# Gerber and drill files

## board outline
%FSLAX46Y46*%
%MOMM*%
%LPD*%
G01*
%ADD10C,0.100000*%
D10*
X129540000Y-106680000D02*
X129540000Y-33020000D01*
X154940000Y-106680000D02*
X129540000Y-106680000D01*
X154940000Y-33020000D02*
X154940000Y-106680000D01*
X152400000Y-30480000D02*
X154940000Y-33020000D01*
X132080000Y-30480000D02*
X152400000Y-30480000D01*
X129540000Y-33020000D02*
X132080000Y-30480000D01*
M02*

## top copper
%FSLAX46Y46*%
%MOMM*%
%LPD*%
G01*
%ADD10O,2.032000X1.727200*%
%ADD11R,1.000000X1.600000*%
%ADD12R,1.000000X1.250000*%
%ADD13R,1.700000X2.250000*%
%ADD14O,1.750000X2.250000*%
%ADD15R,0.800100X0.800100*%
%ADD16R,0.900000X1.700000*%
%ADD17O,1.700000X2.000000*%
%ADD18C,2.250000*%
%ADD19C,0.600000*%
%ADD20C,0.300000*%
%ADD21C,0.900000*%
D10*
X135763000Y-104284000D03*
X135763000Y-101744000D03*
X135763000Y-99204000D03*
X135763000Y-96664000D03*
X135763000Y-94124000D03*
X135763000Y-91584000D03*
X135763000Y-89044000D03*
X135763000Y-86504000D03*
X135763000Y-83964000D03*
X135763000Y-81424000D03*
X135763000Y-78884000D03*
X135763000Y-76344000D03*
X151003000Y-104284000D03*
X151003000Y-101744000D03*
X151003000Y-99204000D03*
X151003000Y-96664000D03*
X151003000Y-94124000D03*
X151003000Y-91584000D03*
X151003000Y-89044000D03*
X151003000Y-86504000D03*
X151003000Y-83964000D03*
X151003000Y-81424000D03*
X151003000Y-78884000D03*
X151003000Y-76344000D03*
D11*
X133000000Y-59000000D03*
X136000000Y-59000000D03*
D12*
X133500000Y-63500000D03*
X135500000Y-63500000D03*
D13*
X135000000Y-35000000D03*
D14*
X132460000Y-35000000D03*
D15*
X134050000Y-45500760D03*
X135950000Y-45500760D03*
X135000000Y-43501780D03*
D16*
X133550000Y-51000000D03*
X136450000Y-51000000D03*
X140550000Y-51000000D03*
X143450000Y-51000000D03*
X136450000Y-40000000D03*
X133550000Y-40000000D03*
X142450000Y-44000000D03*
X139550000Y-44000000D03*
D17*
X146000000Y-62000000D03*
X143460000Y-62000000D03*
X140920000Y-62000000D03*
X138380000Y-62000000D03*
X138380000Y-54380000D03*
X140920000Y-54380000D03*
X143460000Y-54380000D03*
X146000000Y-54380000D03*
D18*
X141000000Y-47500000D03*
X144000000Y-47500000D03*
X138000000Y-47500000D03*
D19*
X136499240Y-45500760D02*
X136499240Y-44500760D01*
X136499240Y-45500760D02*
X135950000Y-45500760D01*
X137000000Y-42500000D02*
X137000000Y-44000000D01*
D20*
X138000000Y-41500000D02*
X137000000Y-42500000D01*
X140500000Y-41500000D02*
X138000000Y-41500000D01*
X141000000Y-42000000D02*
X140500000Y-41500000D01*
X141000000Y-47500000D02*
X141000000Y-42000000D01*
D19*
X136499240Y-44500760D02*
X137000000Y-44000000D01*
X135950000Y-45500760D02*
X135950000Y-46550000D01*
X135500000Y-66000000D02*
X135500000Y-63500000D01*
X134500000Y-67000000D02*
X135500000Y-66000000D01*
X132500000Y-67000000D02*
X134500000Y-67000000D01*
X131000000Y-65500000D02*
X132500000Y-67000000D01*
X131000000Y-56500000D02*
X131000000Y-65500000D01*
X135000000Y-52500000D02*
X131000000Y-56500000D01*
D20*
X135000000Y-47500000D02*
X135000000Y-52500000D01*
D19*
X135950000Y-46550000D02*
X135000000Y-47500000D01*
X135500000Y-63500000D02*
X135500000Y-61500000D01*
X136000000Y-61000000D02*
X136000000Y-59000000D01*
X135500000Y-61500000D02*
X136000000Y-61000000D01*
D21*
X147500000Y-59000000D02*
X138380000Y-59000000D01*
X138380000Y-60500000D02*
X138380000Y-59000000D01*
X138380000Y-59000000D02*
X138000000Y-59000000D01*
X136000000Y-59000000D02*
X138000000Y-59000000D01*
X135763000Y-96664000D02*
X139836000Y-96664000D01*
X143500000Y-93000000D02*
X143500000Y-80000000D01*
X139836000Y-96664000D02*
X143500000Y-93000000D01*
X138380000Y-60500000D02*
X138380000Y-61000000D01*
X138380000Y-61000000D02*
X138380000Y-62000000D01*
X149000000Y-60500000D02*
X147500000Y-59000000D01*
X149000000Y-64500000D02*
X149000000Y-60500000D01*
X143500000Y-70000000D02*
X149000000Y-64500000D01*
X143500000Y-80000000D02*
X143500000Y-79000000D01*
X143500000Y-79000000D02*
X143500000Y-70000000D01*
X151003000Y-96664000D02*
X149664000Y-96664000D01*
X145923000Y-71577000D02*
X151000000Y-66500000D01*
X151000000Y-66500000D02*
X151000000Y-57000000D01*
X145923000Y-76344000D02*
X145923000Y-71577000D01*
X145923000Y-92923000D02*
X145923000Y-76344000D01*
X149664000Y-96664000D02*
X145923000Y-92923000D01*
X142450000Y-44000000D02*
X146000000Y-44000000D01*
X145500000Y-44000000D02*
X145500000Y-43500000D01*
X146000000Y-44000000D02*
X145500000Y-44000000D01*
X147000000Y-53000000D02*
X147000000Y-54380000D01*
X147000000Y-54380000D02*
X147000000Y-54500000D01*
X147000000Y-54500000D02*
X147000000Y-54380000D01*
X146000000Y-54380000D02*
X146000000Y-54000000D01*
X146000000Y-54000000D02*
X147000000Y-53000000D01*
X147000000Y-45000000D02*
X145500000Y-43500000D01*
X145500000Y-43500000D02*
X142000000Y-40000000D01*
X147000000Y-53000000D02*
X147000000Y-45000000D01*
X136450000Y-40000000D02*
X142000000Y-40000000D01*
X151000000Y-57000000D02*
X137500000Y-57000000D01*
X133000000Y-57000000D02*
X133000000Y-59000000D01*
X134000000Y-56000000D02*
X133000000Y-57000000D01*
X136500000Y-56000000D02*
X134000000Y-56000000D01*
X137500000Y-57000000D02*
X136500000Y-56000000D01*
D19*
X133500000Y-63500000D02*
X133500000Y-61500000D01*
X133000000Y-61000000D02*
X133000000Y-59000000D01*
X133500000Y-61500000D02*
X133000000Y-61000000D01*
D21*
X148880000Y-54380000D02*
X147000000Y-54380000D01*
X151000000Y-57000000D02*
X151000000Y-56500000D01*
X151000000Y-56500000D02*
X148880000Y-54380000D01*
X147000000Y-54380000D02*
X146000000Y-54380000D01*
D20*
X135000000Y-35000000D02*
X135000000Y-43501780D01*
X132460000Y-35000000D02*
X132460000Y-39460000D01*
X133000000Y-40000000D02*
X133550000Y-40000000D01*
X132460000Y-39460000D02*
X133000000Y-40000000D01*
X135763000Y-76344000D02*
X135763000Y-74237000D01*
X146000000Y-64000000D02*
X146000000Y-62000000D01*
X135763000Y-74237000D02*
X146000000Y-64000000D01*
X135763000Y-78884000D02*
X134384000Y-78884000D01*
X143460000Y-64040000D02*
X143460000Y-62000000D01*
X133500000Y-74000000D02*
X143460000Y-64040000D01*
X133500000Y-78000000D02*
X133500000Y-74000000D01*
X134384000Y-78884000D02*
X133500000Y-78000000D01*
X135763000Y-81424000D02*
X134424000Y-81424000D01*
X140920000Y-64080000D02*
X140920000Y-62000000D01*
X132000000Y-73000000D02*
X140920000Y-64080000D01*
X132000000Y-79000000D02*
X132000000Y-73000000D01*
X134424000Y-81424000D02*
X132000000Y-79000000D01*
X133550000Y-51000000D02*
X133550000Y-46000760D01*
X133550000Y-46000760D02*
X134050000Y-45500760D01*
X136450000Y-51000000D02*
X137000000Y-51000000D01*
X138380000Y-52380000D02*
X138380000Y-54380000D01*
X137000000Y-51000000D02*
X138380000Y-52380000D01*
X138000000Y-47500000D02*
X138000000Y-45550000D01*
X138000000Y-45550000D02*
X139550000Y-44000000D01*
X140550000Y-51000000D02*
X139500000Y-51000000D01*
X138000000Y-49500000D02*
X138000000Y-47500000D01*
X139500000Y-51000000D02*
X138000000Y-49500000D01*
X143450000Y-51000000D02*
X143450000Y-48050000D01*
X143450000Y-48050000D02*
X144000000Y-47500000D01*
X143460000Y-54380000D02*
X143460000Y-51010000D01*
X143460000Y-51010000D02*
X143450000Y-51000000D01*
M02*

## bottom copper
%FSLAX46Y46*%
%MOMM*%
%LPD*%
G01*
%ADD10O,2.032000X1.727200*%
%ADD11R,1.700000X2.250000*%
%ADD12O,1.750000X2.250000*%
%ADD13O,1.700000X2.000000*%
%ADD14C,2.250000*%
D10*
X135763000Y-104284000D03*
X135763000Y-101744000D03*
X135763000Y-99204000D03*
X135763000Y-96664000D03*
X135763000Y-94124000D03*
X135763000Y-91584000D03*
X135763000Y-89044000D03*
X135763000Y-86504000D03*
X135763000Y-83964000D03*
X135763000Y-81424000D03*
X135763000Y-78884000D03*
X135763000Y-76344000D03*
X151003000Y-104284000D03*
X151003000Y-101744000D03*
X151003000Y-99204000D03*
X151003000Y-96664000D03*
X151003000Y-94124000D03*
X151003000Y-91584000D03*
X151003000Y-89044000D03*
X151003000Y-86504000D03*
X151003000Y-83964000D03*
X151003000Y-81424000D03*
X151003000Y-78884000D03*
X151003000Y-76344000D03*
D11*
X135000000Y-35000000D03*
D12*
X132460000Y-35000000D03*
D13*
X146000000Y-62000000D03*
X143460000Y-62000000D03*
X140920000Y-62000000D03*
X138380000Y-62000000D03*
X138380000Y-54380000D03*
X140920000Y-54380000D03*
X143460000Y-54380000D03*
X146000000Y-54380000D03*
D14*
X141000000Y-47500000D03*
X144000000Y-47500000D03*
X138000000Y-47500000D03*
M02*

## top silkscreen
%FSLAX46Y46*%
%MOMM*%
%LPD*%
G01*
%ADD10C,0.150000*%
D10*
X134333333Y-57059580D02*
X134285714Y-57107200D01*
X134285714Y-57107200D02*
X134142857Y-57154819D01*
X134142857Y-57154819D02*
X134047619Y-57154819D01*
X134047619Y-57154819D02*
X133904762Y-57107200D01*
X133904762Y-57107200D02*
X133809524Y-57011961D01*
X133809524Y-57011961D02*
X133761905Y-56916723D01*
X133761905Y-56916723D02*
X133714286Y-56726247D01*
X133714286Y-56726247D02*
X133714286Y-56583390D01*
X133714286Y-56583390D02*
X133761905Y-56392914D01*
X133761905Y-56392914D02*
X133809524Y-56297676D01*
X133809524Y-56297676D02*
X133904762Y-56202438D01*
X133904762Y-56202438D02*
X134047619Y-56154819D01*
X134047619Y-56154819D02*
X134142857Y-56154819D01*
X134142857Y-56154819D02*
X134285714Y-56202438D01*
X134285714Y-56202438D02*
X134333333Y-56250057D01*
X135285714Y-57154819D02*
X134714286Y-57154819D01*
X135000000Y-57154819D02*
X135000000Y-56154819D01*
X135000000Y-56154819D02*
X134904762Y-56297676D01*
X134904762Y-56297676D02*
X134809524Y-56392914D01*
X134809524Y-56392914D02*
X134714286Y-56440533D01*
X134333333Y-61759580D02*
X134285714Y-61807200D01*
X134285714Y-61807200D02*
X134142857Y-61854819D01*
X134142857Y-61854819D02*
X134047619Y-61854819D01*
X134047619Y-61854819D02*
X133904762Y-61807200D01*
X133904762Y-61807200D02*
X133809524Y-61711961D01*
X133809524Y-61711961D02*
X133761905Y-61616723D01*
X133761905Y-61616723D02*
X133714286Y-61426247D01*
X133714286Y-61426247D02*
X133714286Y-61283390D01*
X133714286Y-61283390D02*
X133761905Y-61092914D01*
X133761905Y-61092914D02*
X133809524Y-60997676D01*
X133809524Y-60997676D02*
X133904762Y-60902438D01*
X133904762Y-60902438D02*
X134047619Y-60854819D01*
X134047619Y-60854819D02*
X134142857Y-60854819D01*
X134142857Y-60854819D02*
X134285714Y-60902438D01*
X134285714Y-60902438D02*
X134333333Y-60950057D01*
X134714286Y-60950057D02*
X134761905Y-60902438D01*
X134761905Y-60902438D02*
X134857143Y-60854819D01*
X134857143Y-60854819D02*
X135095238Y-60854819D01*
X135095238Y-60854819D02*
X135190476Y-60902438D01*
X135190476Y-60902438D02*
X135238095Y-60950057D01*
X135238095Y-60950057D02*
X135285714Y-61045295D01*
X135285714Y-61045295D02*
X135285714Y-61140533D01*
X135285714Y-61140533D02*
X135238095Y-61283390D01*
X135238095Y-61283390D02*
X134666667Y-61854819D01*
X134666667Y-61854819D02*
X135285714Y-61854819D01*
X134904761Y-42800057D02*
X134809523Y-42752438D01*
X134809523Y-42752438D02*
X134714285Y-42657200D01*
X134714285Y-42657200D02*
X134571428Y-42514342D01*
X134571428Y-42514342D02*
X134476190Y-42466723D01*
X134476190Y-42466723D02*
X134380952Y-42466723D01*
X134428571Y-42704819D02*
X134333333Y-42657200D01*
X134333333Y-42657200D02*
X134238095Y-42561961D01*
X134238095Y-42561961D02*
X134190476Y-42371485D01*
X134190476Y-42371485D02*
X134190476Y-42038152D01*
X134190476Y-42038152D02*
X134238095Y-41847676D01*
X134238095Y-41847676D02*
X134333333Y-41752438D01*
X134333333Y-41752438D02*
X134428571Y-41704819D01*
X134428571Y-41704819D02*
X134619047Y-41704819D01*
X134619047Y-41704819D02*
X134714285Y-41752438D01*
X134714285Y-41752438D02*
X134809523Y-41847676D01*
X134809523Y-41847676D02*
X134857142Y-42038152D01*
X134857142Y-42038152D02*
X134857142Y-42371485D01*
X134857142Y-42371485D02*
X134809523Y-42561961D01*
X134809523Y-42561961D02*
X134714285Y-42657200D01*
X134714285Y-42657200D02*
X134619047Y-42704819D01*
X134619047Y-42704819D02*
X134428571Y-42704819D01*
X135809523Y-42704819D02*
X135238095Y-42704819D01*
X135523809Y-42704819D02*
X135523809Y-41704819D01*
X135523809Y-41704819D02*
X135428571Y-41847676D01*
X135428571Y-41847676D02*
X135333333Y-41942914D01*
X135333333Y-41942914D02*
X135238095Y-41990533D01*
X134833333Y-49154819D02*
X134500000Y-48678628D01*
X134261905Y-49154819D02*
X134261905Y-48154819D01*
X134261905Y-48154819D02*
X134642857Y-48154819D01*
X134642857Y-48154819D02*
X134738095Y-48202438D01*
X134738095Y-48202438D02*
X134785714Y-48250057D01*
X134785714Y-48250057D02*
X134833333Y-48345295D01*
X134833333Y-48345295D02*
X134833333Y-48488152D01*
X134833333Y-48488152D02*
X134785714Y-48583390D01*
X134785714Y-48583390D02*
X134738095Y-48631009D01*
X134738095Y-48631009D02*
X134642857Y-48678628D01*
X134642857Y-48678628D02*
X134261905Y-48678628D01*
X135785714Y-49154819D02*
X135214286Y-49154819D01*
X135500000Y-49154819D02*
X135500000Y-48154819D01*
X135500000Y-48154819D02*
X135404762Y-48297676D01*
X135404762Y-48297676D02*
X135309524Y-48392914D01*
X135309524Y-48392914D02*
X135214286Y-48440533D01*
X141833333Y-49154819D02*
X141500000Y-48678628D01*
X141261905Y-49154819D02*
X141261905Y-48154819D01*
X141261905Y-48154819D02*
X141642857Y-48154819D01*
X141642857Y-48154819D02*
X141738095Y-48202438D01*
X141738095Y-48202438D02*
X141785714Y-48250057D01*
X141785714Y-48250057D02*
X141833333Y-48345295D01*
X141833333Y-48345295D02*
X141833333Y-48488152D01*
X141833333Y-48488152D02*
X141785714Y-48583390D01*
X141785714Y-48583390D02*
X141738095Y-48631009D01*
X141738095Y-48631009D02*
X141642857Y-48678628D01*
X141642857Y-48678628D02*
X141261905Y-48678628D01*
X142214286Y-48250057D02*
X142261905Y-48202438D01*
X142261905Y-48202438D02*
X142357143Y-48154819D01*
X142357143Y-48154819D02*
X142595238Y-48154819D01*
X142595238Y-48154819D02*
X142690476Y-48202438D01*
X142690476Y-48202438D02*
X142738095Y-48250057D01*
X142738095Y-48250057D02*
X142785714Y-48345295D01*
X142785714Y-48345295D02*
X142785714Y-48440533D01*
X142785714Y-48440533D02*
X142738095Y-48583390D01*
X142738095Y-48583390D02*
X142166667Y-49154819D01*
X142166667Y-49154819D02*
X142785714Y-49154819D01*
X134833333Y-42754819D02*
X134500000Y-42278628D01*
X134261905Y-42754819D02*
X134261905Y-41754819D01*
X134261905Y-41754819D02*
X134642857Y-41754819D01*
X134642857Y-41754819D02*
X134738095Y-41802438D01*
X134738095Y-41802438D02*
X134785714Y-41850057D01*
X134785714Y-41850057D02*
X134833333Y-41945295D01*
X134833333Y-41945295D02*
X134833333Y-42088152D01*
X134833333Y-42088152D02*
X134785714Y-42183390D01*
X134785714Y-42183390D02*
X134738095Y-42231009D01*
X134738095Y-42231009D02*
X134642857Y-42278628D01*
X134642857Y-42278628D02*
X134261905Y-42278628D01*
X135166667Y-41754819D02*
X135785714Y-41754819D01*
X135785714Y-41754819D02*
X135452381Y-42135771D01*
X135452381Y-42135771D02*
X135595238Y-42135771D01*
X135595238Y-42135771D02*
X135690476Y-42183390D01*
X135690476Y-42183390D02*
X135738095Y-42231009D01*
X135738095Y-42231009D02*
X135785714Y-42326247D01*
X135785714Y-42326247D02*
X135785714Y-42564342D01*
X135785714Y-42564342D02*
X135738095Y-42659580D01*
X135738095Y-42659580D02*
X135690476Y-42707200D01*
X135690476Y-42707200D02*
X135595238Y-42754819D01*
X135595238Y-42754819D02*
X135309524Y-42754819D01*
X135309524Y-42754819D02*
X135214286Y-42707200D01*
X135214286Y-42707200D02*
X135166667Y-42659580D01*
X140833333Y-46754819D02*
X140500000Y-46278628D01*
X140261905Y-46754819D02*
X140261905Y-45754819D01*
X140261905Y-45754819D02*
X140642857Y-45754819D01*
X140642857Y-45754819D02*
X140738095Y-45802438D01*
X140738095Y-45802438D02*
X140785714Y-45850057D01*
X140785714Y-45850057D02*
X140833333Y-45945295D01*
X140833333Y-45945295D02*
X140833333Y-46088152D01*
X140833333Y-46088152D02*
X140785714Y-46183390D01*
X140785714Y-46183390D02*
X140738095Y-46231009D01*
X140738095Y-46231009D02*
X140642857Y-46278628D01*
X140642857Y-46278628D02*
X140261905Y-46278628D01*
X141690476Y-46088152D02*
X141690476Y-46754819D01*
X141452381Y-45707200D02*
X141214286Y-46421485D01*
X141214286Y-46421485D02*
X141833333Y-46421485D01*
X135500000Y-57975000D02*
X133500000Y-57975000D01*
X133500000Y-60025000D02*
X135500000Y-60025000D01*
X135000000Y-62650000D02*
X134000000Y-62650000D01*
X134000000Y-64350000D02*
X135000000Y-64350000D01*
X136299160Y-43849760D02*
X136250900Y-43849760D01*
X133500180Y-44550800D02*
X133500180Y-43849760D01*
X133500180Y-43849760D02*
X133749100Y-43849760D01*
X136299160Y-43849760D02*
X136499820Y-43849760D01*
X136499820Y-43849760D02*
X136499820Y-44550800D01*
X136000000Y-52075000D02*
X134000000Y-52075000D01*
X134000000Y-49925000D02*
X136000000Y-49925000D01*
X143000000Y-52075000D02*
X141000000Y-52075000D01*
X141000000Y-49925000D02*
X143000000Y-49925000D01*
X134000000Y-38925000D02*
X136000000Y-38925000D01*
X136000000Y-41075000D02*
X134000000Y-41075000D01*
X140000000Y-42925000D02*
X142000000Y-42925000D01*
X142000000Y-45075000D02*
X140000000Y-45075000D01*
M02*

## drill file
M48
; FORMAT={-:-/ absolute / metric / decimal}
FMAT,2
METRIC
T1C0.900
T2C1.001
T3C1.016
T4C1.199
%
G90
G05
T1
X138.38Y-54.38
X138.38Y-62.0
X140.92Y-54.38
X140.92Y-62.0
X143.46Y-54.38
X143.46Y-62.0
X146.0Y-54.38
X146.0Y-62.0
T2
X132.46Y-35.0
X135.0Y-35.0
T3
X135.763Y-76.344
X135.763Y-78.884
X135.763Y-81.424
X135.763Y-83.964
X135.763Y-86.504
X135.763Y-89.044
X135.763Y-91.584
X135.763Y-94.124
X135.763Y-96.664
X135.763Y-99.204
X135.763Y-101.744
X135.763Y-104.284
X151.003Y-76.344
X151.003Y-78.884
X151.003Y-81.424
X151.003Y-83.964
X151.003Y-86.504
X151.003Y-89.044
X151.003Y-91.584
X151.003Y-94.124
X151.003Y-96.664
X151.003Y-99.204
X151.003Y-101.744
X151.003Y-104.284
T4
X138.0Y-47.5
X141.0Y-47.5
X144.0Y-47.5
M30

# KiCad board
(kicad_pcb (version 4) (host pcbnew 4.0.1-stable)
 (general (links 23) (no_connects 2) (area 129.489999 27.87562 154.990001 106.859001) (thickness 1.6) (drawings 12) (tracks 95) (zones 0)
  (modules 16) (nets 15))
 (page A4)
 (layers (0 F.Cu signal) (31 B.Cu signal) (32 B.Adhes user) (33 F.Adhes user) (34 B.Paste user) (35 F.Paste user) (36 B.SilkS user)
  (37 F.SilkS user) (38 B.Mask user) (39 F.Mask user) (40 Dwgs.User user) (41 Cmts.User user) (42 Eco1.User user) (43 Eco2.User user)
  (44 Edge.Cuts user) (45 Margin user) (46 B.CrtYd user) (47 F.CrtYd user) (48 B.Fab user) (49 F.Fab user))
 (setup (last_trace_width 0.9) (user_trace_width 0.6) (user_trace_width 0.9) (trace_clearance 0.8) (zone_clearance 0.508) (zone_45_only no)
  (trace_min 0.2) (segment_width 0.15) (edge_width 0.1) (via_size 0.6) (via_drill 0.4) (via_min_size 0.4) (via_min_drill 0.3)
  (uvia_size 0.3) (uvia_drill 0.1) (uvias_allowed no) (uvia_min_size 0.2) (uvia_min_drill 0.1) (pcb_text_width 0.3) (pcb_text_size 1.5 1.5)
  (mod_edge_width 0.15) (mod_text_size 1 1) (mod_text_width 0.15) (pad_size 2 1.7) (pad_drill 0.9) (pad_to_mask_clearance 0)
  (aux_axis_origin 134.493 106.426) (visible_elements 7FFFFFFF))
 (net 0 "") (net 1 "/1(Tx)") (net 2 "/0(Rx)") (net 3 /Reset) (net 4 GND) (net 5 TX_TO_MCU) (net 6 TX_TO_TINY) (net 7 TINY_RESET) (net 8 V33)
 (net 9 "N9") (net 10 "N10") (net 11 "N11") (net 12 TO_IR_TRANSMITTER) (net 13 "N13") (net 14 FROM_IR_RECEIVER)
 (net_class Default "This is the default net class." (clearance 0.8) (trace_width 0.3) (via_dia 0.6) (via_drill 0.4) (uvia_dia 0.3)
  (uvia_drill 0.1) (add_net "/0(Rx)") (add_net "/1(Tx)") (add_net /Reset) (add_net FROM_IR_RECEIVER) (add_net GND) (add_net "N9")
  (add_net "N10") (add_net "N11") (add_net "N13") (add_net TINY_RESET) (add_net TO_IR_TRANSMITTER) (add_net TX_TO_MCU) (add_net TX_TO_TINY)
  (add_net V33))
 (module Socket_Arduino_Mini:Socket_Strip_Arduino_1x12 (layer B.Cu) (at 135.763 104.284 90)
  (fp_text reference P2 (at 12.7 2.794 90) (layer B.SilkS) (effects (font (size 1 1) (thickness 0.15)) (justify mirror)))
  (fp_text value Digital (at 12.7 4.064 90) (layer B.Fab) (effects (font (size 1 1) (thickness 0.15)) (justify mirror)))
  (pad 1 thru_hole oval (at 0 0 90) (size 1.7272 2.032) (drill 1.016) (layers *.Cu *.Mask B.SilkS) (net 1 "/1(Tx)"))
  (pad 2 thru_hole oval (at 2.54 0 90) (size 1.7272 2.032) (drill 1.016) (layers *.Cu *.Mask B.SilkS) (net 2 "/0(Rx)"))
  (pad 3 thru_hole oval (at 5.08 0 90) (size 1.7272 2.032) (drill 1.016) (layers *.Cu *.Mask B.SilkS) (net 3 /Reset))
  (pad 4 thru_hole oval (at 7.62 0 90) (size 1.7272 2.032) (drill 1.016) (layers *.Cu *.Mask B.SilkS) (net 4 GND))
  (pad 5 thru_hole oval (at 10.16 0 90) (size 1.7272 2.032) (drill 1.016) (layers *.Cu *.Mask B.SilkS))
  (pad 6 thru_hole oval (at 12.7 0 90) (size 1.7272 2.032) (drill 1.016) (layers *.Cu *.Mask B.SilkS))
  (pad 7 thru_hole oval (at 15.24 0 90) (size 1.7272 2.032) (drill 1.016) (layers *.Cu *.Mask B.SilkS))
  (pad 8 thru_hole oval (at 17.78 0 90) (size 1.7272 2.032) (drill 1.016) (layers *.Cu *.Mask B.SilkS))
  (pad 9 thru_hole oval (at 20.32 0 90) (size 1.7272 2.032) (drill 1.016) (layers *.Cu *.Mask B.SilkS))
  (pad 10 thru_hole oval (at 22.86 0 90) (size 1.7272 2.032) (drill 1.016) (layers *.Cu *.Mask B.SilkS) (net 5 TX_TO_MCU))
  (pad 11 thru_hole oval (at 25.4 0 90) (size 1.7272 2.032) (drill 1.016) (layers *.Cu *.Mask B.SilkS) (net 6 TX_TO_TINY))
  (pad 12 thru_hole oval (at 27.94 0 90) (size 1.7272 2.032) (drill 1.016) (layers *.Cu *.Mask B.SilkS) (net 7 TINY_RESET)))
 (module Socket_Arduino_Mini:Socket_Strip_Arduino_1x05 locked (layer B.Cu) (at 138.303 104.284)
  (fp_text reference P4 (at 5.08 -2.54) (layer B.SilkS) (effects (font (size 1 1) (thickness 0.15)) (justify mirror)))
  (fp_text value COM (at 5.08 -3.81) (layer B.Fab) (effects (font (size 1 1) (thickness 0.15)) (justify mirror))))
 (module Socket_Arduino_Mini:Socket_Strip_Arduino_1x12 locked (layer B.Cu) (at 151.003 104.284 90)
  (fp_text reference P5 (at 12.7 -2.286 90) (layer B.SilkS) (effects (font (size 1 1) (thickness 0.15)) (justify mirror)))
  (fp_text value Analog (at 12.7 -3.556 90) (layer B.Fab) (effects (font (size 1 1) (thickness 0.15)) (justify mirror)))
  (pad 1 thru_hole oval (at 0 0 90) (size 1.7272 2.032) (drill 1.016) (layers *.Cu *.Mask B.SilkS))
  (pad 2 thru_hole oval (at 2.54 0 90) (size 1.7272 2.032) (drill 1.016) (layers *.Cu *.Mask B.SilkS) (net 4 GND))
  (pad 3 thru_hole oval (at 5.08 0 90) (size 1.7272 2.032) (drill 1.016) (layers *.Cu *.Mask B.SilkS) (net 3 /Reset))
  (pad 4 thru_hole oval (at 7.62 0 90) (size 1.7272 2.032) (drill 1.016) (layers *.Cu *.Mask B.SilkS) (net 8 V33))
  (pad 5 thru_hole oval (at 10.16 0 90) (size 1.7272 2.032) (drill 1.016) (layers *.Cu *.Mask B.SilkS))
  (pad 6 thru_hole oval (at 12.7 0 90) (size 1.7272 2.032) (drill 1.016) (layers *.Cu *.Mask B.SilkS))
  (pad 7 thru_hole oval (at 15.24 0 90) (size 1.7272 2.032) (drill 1.016) (layers *.Cu *.Mask B.SilkS))
  (pad 8 thru_hole oval (at 17.78 0 90) (size 1.7272 2.032) (drill 1.016) (layers *.Cu *.Mask B.SilkS))
  (pad 9 thru_hole oval (at 20.32 0 90) (size 1.7272 2.032) (drill 1.016) (layers *.Cu *.Mask B.SilkS))
  (pad 10 thru_hole oval (at 22.86 0 90) (size 1.7272 2.032) (drill 1.016) (layers *.Cu *.Mask B.SilkS))
  (pad 11 thru_hole oval (at 25.4 0 90) (size 1.7272 2.032) (drill 1.016) (layers *.Cu *.Mask B.SilkS))
  (pad 12 thru_hole oval (at 27.94 0 90) (size 1.7272 2.032) (drill 1.016) (layers *.Cu *.Mask B.SilkS)))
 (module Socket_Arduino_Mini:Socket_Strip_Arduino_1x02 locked (layer B.Cu) (at 138.303 78.884 90)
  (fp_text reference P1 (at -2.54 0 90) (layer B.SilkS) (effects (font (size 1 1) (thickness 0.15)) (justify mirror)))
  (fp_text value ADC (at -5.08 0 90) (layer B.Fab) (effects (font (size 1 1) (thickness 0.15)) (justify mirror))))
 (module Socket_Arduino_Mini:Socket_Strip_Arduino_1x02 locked (layer B.Cu) (at 140.843 78.884 90)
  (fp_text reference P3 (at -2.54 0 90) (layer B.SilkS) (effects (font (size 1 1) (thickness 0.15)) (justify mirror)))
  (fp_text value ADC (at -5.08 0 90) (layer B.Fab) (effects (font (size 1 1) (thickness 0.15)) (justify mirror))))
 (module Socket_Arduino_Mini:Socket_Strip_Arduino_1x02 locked (layer B.Cu) (at 145.923 76.344)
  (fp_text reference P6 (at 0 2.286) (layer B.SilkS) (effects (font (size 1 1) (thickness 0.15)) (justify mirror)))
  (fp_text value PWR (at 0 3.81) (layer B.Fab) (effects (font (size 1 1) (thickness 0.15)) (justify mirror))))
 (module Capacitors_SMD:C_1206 (layer F.Cu) (at 134.5 59)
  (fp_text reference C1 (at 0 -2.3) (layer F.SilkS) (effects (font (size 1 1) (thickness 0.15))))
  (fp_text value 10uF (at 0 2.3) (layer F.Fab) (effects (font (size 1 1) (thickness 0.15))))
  (fp_line (start 1 -1.025) (end -1 -1.025) (layer F.SilkS) (width 0.15))
  (fp_line (start -1 1.025) (end 1 1.025) (layer F.SilkS) (width 0.15))
  (pad 1 smd rect (at -1.5 0) (size 1 1.6) (layers F.Cu F.Paste F.Mask) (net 8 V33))
  (pad 2 smd rect (at 1.5 0) (size 1 1.6) (layers F.Cu F.Paste F.Mask) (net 4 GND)))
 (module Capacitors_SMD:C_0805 (layer F.Cu) (at 134.5 63.5)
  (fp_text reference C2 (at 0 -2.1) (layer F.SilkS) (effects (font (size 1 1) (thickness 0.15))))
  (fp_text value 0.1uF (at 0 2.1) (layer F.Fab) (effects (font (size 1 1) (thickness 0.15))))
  (fp_line (start 0.5 -0.85) (end -0.5 -0.85) (layer F.SilkS) (width 0.15))
  (fp_line (start -0.5 0.85) (end 0.5 0.85) (layer F.SilkS) (width 0.15))
  (pad 1 smd rect (at -1 0) (size 1 1.25) (layers F.Cu F.Paste F.Mask) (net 8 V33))
  (pad 2 smd rect (at 1 0) (size 1 1.25) (layers F.Cu F.Paste F.Mask) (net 4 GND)))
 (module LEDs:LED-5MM (layer B.Cu) (at 135 35 180)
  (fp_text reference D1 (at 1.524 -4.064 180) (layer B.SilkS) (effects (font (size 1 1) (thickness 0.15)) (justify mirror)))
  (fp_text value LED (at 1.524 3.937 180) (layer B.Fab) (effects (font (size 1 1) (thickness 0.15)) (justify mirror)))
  (pad 1 thru_hole rect (at 0 0 90) (size 2.25 1.7) (drill 1.00076) (layers *.Cu *.Mask B.SilkS) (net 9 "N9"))
  (pad 2 thru_hole oval (at 2.54 0 180) (size 1.75 2.25) (drill 1.00076) (layers *.Cu *.Mask B.SilkS) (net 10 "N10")))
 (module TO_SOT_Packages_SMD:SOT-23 (layer F.Cu) (at 135 44.5)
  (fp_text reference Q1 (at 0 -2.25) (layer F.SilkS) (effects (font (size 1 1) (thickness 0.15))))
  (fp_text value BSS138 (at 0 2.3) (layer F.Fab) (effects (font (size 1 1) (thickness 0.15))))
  (fp_line (start 1.29916 -0.65024) (end 1.2509 -0.65024) (layer F.SilkS) (width 0.15))
  (fp_line (start -1.49982 0.0508) (end -1.49982 -0.65024) (layer F.SilkS) (width 0.15))
  (fp_line (start -1.49982 -0.65024) (end -1.2509 -0.65024) (layer F.SilkS) (width 0.15))
  (fp_line (start 1.29916 -0.65024) (end 1.49982 -0.65024) (layer F.SilkS) (width 0.15))
  (fp_line (start 1.49982 -0.65024) (end 1.49982 0.0508) (layer F.SilkS) (width 0.15))
  (pad 1 smd rect (at -0.95 1.00076) (size 0.8001 0.8001) (layers F.Cu F.Paste F.Mask) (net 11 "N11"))
  (pad 2 smd rect (at 0.95 1.00076) (size 0.8001 0.8001) (layers F.Cu F.Paste F.Mask) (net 4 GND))
  (pad 3 smd rect (at 0 -0.99822) (size 0.8001 0.8001) (layers F.Cu F.Paste F.Mask) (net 9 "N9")))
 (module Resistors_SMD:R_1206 (layer F.Cu) (at 135 51)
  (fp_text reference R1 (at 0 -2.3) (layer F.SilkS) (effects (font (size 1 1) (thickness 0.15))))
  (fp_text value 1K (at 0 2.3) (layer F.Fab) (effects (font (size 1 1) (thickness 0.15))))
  (fp_line (start 1 1.075) (end -1 1.075) (layer F.SilkS) (width 0.15))
  (fp_line (start -1 -1.075) (end 1 -1.075) (layer F.SilkS) (width 0.15))
  (pad 1 smd rect (at -1.45 0) (size 0.9 1.7) (layers F.Cu F.Paste F.Mask) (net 11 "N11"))
  (pad 2 smd rect (at 1.45 0) (size 0.9 1.7) (layers F.Cu F.Paste F.Mask) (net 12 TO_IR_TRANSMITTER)))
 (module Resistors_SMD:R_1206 (layer F.Cu) (at 142 51)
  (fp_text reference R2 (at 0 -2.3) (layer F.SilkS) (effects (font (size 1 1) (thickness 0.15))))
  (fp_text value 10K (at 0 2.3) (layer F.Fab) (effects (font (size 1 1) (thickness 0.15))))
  (fp_line (start 1 1.075) (end -1 1.075) (layer F.SilkS) (width 0.15))
  (fp_line (start -1 -1.075) (end 1 -1.075) (layer F.SilkS) (width 0.15))
  (pad 1 smd rect (at -1.45 0) (size 0.9 1.7) (layers F.Cu F.Paste F.Mask) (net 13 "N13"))
  (pad 2 smd rect (at 1.45 0) (size 0.9 1.7) (layers F.Cu F.Paste F.Mask) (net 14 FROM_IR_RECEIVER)))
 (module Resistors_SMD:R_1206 (layer F.Cu) (at 135 40 180)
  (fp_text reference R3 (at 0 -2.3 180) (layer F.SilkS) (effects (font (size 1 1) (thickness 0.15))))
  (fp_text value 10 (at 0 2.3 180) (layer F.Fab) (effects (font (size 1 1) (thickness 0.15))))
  (fp_line (start 1 1.075) (end -1 1.075) (layer F.SilkS) (width 0.15))
  (fp_line (start -1 -1.075) (end 1 -1.075) (layer F.SilkS) (width 0.15))
  (pad 1 smd rect (at -1.45 0 180) (size 0.9 1.7) (layers F.Cu F.Paste F.Mask) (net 8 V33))
  (pad 2 smd rect (at 1.45 0 180) (size 0.9 1.7) (layers F.Cu F.Paste F.Mask) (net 10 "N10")))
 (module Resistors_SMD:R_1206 (layer F.Cu) (at 141 44 180)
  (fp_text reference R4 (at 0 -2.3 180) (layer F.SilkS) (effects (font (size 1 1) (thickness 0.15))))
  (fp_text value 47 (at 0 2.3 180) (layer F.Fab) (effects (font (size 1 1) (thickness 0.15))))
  (fp_line (start 1 1.075) (end -1 1.075) (layer F.SilkS) (width 0.15))
  (fp_line (start -1 -1.075) (end 1 -1.075) (layer F.SilkS) (width 0.15))
  (pad 1 smd rect (at -1.45 0 180) (size 0.9 1.7) (layers F.Cu F.Paste F.Mask) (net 8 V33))
  (pad 2 smd rect (at 1.45 0 180) (size 0.9 1.7) (layers F.Cu F.Paste F.Mask) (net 13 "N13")))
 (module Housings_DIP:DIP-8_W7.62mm (layer B.Cu) (at 146 62 90)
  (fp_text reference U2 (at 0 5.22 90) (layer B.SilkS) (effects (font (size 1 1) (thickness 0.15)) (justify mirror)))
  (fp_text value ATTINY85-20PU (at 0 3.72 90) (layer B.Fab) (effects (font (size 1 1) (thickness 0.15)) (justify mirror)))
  (pad 1 thru_hole oval (at 0 0 90) (size 2 1.7) (drill 0.9) (layers *.Cu *.Mask B.SilkS) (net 7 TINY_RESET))
  (pad 2 thru_hole oval (at 0 -2.54 90) (size 2 1.7) (drill 0.9) (layers *.Cu *.Mask B.SilkS) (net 6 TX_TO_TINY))
  (pad 3 thru_hole oval (at 0 -5.08 90) (size 2 1.7) (drill 0.9) (layers *.Cu *.Mask B.SilkS) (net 5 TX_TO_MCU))
  (pad 4 thru_hole oval (at 0 -7.62 90) (size 2 1.7) (drill 0.9) (layers *.Cu *.Mask B.SilkS) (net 4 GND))
  (pad 5 thru_hole oval (at 7.62 -7.62 90) (size 2 1.7) (drill 0.9) (layers *.Cu *.Mask B.SilkS) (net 12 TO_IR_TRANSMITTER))
  (pad 6 thru_hole oval (at 7.62 -5.08 90) (size 2 1.7) (drill 0.9) (layers *.Cu *.Mask B.SilkS))
  (pad 7 thru_hole oval (at 7.62 -2.54 90) (size 2 1.7) (drill 0.9) (layers *.Cu *.Mask B.SilkS) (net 14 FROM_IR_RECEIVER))
  (pad 8 thru_hole oval (at 7.62 0 90) (size 2 1.7) (drill 0.9) (layers *.Cu *.Mask B.SilkS) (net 8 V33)))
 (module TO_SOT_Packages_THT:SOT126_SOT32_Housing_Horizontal (layer B.Cu) (at 141 47.5 180)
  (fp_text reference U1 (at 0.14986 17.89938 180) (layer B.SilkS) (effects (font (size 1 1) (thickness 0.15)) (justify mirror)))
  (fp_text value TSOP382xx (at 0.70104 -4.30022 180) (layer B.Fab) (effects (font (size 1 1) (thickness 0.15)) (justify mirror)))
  (pad 2 thru_hole circle (at 0 0 180) (size 2.25 2.25) (drill 1.19888) (layers *.Cu *.Mask B.SilkS) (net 4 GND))
  (pad 1 thru_hole circle (at -3 0 180) (size 2.25 2.25) (drill 1.19888) (layers *.Cu *.Mask B.SilkS) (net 14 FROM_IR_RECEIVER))
  (pad 3 thru_hole circle (at 3 0 180) (size 2.25 2.25) (drill 1.19888) (layers *.Cu *.Mask B.SilkS) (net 13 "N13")))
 (gr_line (start 129.54 106.68) (end 129.54 33.02) (angle 90) (layer Edge.Cuts) (width 0.1))
 (gr_line (start 154.94 106.68) (end 129.54 106.68) (angle 90) (layer Edge.Cuts) (width 0.1))
 (gr_line (start 154.94 33.02) (end 154.94 106.68) (angle 90) (layer Edge.Cuts) (width 0.1))
 (gr_line (start 152.4 30.48) (end 154.94 33.02) (angle 90) (layer Edge.Cuts) (width 0.1))
 (gr_line (start 132.08 30.48) (end 152.4 30.48) (angle 90) (layer Edge.Cuts) (width 0.1))
 (gr_line (start 129.54 33.02) (end 132.08 30.48) (angle 90) (layer Edge.Cuts) (width 0.1))
 (segment (start 136.49924 45.50076) (end 136.49924 44.50076) (width 0.6) (layer F.Cu) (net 4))
 (segment (start 136.49924 45.50076) (end 135.95 45.50076) (width 0.6) (layer F.Cu) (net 4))
 (segment (start 137 42.5) (end 137 44) (width 0.6) (layer F.Cu) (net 4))
 (segment (start 138 41.5) (end 137 42.5) (width 0.3) (layer F.Cu) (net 4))
 (segment (start 140.5 41.5) (end 138 41.5) (width 0.3) (layer F.Cu) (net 4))
 (segment (start 141 42) (end 140.5 41.5) (width 0.3) (layer F.Cu) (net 4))
 (segment (start 141 47.5) (end 141 42) (width 0.3) (layer F.Cu) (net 4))
 (segment (start 136.49924 44.50076) (end 137 44) (width 0.6) (layer F.Cu) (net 4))
 (segment (start 135.95 45.50076) (end 135.95 46.55) (width 0.6) (layer F.Cu) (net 4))
 (segment (start 135.5 66) (end 135.5 63.5) (width 0.6) (layer F.Cu) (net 4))
 (segment (start 134.5 67) (end 135.5 66) (width 0.6) (layer F.Cu) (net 4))
 (segment (start 132.5 67) (end 134.5 67) (width 0.6) (layer F.Cu) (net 4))
 (segment (start 131 65.5) (end 132.5 67) (width 0.6) (layer F.Cu) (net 4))
 (segment (start 131 56.5) (end 131 65.5) (width 0.6) (layer F.Cu) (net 4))
 (segment (start 135 52.5) (end 131 56.5) (width 0.6) (layer F.Cu) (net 4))
 (segment (start 135 47.5) (end 135 52.5) (width 0.3) (layer F.Cu) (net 4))
 (segment (start 135.95 46.55) (end 135 47.5) (width 0.6) (layer F.Cu) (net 4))
 (segment (start 135.5 63.5) (end 135.5 61.5) (width 0.6) (layer F.Cu) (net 4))
 (segment (start 136 61) (end 136 59) (width 0.6) (layer F.Cu) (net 4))
 (segment (start 135.5 61.5) (end 136 61) (width 0.6) (layer F.Cu) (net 4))
 (segment (start 147.5 59) (end 138.38 59) (width 0.9) (layer F.Cu) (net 4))
 (segment (start 138.38 60.5) (end 138.38 59) (width 0.9) (layer F.Cu) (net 4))
 (segment (start 138.38 59) (end 138 59) (width 0.9) (layer F.Cu) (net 4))
 (segment (start 136 59) (end 138 59) (width 0.9) (layer F.Cu) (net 4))
 (segment (start 135.763 96.664) (end 139.836 96.664) (width 0.9) (layer F.Cu) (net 4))
 (segment (start 143.5 93) (end 143.5 80) (width 0.9) (layer F.Cu) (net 4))
 (segment (start 139.836 96.664) (end 143.5 93) (width 0.9) (layer F.Cu) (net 4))
 (segment (start 138.38 60.5) (end 138.38 61) (width 0.9) (layer F.Cu) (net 4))
 (segment (start 138.38 61) (end 138.38 62) (width 0.9) (layer F.Cu) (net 4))
 (segment (start 149 60.5) (end 147.5 59) (width 0.9) (layer F.Cu) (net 4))
 (segment (start 149 64.5) (end 149 60.5) (width 0.9) (layer F.Cu) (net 4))
 (segment (start 143.5 70) (end 149 64.5) (width 0.9) (layer F.Cu) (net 4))
 (segment (start 143.5 80) (end 143.5 79) (width 0.9) (layer F.Cu) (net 4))
 (segment (start 143.5 79) (end 143.5 70) (width 0.9) (layer F.Cu) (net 4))
 (segment (start 151.003 96.664) (end 149.664 96.664) (width 0.9) (layer F.Cu) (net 8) (status 400000))
 (segment (start 145.923 71.577) (end 151 66.5) (width 0.9) (layer F.Cu) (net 8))
 (segment (start 151 66.5) (end 151 57) (width 0.9) (layer F.Cu) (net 8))
 (segment (start 145.923 76.344) (end 145.923 71.577) (width 0.9) (layer F.Cu) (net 8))
 (segment (start 145.923 92.923) (end 145.923 76.344) (width 0.9) (layer F.Cu) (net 8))
 (segment (start 149.664 96.664) (end 145.923 92.923) (width 0.9) (layer F.Cu) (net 8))
 (segment (start 142.45 44) (end 146 44) (width 0.9) (layer F.Cu) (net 8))
 (segment (start 145.5 44) (end 145.5 43.5) (width 0.9) (layer F.Cu) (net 8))
 (segment (start 146 44) (end 145.5 44) (width 0.9) (layer F.Cu) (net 8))
 (segment (start 147 53) (end 147 54.38) (width 0.9) (layer F.Cu) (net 8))
 (segment (start 147 54.38) (end 147 54.5) (width 0.9) (layer F.Cu) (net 8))
 (segment (start 147 54.5) (end 147 54.38) (width 0.9) (layer F.Cu) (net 8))
 (segment (start 146 54.38) (end 146 54) (width 0.9) (layer F.Cu) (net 8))
 (segment (start 146 54) (end 147 53) (width 0.9) (layer F.Cu) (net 8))
 (segment (start 147 45) (end 145.5 43.5) (width 0.9) (layer F.Cu) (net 8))
 (segment (start 145.5 43.5) (end 142 40) (width 0.9) (layer F.Cu) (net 8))
 (segment (start 147 53) (end 147 45) (width 0.9) (layer F.Cu) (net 8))
 (segment (start 136.45 40) (end 142 40) (width 0.9) (layer F.Cu) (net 8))
 (segment (start 151 57) (end 137.5 57) (width 0.9) (layer F.Cu) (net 8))
 (segment (start 133 57) (end 133 59) (width 0.9) (layer F.Cu) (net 8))
 (segment (start 134 56) (end 133 57) (width 0.9) (layer F.Cu) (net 8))
 (segment (start 136.5 56) (end 134 56) (width 0.9) (layer F.Cu) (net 8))
 (segment (start 137.5 57) (end 136.5 56) (width 0.9) (layer F.Cu) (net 8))
 (segment (start 133.5 63.5) (end 133.5 61.5) (width 0.6) (layer F.Cu) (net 8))
 (segment (start 133 61) (end 133 59) (width 0.6) (layer F.Cu) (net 8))
 (segment (start 133.5 61.5) (end 133 61) (width 0.6) (layer F.Cu) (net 8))
 (segment (start 148.88 54.38) (end 147 54.38) (width 0.9) (layer F.Cu) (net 8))
 (segment (start 151 57) (end 151 56.5) (width 0.9) (layer F.Cu) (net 8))
 (segment (start 151 56.5) (end 148.88 54.38) (width 0.9) (layer F.Cu) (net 8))
 (segment (start 147 54.38) (end 146 54.38) (width 0.9) (layer F.Cu) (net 8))
 (segment (start 135 35) (end 135 43.50178) (width 0.3) (layer F.Cu) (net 9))
 (segment (start 132.46 35) (end 132.46 39.46) (width 0.3) (layer F.Cu) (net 10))
 (segment (start 133 40) (end 133.55 40) (width 0.3) (layer F.Cu) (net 10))
 (segment (start 132.46 39.46) (end 133 40) (width 0.3) (layer F.Cu) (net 10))
 (segment (start 135.763 76.344) (end 135.763 74.237) (width 0.3) (layer F.Cu) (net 7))
 (segment (start 146 64) (end 146 62) (width 0.3) (layer F.Cu) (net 7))
 (segment (start 135.763 74.237) (end 146 64) (width 0.3) (layer F.Cu) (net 7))
 (segment (start 135.763 78.884) (end 134.384 78.884) (width 0.3) (layer F.Cu) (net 6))
 (segment (start 143.46 64.04) (end 143.46 62) (width 0.3) (layer F.Cu) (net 6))
 (segment (start 133.5 74) (end 143.46 64.04) (width 0.3) (layer F.Cu) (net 6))
 (segment (start 133.5 78) (end 133.5 74) (width 0.3) (layer F.Cu) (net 6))
 (segment (start 134.384 78.884) (end 133.5 78) (width 0.3) (layer F.Cu) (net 6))
 (segment (start 135.763 81.424) (end 134.424 81.424) (width 0.3) (layer F.Cu) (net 5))
 (segment (start 140.92 64.08) (end 140.92 62) (width 0.3) (layer F.Cu) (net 5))
 (segment (start 132 73) (end 140.92 64.08) (width 0.3) (layer F.Cu) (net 5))
 (segment (start 132 79) (end 132 73) (width 0.3) (layer F.Cu) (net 5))
 (segment (start 134.424 81.424) (end 132 79) (width 0.3) (layer F.Cu) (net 5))
 (segment (start 133.55 51) (end 133.55 46.00076) (width 0.3) (layer F.Cu) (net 11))
 (segment (start 133.55 46.00076) (end 134.05 45.50076) (width 0.3) (layer F.Cu) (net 11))
 (segment (start 136.45 51) (end 137 51) (width 0.3) (layer F.Cu) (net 12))
 (segment (start 138.38 52.38) (end 138.38 54.38) (width 0.3) (layer F.Cu) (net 12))
 (segment (start 137 51) (end 138.38 52.38) (width 0.3) (layer F.Cu) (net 12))
 (segment (start 138 47.5) (end 138 45.55) (width 0.3) (layer F.Cu) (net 13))
 (segment (start 138 45.55) (end 139.55 44) (width 0.3) (layer F.Cu) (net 13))
 (segment (start 140.55 51) (end 139.5 51) (width 0.3) (layer F.Cu) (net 13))
 (segment (start 138 49.5) (end 138 47.5) (width 0.3) (layer F.Cu) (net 13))
 (segment (start 139.5 51) (end 138 49.5) (width 0.3) (layer F.Cu) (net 13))
 (segment (start 143.45 51) (end 143.45 48.05) (width 0.3) (layer F.Cu) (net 14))
 (segment (start 143.45 48.05) (end 144 47.5) (width 0.3) (layer F.Cu) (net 14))
 (segment (start 143.46 54.38) (end 143.46 51.01) (width 0.3) (layer F.Cu) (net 14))
 (segment (start 143.46 51.01) (end 143.45 51) (width 0.3) (layer F.Cu) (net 14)))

